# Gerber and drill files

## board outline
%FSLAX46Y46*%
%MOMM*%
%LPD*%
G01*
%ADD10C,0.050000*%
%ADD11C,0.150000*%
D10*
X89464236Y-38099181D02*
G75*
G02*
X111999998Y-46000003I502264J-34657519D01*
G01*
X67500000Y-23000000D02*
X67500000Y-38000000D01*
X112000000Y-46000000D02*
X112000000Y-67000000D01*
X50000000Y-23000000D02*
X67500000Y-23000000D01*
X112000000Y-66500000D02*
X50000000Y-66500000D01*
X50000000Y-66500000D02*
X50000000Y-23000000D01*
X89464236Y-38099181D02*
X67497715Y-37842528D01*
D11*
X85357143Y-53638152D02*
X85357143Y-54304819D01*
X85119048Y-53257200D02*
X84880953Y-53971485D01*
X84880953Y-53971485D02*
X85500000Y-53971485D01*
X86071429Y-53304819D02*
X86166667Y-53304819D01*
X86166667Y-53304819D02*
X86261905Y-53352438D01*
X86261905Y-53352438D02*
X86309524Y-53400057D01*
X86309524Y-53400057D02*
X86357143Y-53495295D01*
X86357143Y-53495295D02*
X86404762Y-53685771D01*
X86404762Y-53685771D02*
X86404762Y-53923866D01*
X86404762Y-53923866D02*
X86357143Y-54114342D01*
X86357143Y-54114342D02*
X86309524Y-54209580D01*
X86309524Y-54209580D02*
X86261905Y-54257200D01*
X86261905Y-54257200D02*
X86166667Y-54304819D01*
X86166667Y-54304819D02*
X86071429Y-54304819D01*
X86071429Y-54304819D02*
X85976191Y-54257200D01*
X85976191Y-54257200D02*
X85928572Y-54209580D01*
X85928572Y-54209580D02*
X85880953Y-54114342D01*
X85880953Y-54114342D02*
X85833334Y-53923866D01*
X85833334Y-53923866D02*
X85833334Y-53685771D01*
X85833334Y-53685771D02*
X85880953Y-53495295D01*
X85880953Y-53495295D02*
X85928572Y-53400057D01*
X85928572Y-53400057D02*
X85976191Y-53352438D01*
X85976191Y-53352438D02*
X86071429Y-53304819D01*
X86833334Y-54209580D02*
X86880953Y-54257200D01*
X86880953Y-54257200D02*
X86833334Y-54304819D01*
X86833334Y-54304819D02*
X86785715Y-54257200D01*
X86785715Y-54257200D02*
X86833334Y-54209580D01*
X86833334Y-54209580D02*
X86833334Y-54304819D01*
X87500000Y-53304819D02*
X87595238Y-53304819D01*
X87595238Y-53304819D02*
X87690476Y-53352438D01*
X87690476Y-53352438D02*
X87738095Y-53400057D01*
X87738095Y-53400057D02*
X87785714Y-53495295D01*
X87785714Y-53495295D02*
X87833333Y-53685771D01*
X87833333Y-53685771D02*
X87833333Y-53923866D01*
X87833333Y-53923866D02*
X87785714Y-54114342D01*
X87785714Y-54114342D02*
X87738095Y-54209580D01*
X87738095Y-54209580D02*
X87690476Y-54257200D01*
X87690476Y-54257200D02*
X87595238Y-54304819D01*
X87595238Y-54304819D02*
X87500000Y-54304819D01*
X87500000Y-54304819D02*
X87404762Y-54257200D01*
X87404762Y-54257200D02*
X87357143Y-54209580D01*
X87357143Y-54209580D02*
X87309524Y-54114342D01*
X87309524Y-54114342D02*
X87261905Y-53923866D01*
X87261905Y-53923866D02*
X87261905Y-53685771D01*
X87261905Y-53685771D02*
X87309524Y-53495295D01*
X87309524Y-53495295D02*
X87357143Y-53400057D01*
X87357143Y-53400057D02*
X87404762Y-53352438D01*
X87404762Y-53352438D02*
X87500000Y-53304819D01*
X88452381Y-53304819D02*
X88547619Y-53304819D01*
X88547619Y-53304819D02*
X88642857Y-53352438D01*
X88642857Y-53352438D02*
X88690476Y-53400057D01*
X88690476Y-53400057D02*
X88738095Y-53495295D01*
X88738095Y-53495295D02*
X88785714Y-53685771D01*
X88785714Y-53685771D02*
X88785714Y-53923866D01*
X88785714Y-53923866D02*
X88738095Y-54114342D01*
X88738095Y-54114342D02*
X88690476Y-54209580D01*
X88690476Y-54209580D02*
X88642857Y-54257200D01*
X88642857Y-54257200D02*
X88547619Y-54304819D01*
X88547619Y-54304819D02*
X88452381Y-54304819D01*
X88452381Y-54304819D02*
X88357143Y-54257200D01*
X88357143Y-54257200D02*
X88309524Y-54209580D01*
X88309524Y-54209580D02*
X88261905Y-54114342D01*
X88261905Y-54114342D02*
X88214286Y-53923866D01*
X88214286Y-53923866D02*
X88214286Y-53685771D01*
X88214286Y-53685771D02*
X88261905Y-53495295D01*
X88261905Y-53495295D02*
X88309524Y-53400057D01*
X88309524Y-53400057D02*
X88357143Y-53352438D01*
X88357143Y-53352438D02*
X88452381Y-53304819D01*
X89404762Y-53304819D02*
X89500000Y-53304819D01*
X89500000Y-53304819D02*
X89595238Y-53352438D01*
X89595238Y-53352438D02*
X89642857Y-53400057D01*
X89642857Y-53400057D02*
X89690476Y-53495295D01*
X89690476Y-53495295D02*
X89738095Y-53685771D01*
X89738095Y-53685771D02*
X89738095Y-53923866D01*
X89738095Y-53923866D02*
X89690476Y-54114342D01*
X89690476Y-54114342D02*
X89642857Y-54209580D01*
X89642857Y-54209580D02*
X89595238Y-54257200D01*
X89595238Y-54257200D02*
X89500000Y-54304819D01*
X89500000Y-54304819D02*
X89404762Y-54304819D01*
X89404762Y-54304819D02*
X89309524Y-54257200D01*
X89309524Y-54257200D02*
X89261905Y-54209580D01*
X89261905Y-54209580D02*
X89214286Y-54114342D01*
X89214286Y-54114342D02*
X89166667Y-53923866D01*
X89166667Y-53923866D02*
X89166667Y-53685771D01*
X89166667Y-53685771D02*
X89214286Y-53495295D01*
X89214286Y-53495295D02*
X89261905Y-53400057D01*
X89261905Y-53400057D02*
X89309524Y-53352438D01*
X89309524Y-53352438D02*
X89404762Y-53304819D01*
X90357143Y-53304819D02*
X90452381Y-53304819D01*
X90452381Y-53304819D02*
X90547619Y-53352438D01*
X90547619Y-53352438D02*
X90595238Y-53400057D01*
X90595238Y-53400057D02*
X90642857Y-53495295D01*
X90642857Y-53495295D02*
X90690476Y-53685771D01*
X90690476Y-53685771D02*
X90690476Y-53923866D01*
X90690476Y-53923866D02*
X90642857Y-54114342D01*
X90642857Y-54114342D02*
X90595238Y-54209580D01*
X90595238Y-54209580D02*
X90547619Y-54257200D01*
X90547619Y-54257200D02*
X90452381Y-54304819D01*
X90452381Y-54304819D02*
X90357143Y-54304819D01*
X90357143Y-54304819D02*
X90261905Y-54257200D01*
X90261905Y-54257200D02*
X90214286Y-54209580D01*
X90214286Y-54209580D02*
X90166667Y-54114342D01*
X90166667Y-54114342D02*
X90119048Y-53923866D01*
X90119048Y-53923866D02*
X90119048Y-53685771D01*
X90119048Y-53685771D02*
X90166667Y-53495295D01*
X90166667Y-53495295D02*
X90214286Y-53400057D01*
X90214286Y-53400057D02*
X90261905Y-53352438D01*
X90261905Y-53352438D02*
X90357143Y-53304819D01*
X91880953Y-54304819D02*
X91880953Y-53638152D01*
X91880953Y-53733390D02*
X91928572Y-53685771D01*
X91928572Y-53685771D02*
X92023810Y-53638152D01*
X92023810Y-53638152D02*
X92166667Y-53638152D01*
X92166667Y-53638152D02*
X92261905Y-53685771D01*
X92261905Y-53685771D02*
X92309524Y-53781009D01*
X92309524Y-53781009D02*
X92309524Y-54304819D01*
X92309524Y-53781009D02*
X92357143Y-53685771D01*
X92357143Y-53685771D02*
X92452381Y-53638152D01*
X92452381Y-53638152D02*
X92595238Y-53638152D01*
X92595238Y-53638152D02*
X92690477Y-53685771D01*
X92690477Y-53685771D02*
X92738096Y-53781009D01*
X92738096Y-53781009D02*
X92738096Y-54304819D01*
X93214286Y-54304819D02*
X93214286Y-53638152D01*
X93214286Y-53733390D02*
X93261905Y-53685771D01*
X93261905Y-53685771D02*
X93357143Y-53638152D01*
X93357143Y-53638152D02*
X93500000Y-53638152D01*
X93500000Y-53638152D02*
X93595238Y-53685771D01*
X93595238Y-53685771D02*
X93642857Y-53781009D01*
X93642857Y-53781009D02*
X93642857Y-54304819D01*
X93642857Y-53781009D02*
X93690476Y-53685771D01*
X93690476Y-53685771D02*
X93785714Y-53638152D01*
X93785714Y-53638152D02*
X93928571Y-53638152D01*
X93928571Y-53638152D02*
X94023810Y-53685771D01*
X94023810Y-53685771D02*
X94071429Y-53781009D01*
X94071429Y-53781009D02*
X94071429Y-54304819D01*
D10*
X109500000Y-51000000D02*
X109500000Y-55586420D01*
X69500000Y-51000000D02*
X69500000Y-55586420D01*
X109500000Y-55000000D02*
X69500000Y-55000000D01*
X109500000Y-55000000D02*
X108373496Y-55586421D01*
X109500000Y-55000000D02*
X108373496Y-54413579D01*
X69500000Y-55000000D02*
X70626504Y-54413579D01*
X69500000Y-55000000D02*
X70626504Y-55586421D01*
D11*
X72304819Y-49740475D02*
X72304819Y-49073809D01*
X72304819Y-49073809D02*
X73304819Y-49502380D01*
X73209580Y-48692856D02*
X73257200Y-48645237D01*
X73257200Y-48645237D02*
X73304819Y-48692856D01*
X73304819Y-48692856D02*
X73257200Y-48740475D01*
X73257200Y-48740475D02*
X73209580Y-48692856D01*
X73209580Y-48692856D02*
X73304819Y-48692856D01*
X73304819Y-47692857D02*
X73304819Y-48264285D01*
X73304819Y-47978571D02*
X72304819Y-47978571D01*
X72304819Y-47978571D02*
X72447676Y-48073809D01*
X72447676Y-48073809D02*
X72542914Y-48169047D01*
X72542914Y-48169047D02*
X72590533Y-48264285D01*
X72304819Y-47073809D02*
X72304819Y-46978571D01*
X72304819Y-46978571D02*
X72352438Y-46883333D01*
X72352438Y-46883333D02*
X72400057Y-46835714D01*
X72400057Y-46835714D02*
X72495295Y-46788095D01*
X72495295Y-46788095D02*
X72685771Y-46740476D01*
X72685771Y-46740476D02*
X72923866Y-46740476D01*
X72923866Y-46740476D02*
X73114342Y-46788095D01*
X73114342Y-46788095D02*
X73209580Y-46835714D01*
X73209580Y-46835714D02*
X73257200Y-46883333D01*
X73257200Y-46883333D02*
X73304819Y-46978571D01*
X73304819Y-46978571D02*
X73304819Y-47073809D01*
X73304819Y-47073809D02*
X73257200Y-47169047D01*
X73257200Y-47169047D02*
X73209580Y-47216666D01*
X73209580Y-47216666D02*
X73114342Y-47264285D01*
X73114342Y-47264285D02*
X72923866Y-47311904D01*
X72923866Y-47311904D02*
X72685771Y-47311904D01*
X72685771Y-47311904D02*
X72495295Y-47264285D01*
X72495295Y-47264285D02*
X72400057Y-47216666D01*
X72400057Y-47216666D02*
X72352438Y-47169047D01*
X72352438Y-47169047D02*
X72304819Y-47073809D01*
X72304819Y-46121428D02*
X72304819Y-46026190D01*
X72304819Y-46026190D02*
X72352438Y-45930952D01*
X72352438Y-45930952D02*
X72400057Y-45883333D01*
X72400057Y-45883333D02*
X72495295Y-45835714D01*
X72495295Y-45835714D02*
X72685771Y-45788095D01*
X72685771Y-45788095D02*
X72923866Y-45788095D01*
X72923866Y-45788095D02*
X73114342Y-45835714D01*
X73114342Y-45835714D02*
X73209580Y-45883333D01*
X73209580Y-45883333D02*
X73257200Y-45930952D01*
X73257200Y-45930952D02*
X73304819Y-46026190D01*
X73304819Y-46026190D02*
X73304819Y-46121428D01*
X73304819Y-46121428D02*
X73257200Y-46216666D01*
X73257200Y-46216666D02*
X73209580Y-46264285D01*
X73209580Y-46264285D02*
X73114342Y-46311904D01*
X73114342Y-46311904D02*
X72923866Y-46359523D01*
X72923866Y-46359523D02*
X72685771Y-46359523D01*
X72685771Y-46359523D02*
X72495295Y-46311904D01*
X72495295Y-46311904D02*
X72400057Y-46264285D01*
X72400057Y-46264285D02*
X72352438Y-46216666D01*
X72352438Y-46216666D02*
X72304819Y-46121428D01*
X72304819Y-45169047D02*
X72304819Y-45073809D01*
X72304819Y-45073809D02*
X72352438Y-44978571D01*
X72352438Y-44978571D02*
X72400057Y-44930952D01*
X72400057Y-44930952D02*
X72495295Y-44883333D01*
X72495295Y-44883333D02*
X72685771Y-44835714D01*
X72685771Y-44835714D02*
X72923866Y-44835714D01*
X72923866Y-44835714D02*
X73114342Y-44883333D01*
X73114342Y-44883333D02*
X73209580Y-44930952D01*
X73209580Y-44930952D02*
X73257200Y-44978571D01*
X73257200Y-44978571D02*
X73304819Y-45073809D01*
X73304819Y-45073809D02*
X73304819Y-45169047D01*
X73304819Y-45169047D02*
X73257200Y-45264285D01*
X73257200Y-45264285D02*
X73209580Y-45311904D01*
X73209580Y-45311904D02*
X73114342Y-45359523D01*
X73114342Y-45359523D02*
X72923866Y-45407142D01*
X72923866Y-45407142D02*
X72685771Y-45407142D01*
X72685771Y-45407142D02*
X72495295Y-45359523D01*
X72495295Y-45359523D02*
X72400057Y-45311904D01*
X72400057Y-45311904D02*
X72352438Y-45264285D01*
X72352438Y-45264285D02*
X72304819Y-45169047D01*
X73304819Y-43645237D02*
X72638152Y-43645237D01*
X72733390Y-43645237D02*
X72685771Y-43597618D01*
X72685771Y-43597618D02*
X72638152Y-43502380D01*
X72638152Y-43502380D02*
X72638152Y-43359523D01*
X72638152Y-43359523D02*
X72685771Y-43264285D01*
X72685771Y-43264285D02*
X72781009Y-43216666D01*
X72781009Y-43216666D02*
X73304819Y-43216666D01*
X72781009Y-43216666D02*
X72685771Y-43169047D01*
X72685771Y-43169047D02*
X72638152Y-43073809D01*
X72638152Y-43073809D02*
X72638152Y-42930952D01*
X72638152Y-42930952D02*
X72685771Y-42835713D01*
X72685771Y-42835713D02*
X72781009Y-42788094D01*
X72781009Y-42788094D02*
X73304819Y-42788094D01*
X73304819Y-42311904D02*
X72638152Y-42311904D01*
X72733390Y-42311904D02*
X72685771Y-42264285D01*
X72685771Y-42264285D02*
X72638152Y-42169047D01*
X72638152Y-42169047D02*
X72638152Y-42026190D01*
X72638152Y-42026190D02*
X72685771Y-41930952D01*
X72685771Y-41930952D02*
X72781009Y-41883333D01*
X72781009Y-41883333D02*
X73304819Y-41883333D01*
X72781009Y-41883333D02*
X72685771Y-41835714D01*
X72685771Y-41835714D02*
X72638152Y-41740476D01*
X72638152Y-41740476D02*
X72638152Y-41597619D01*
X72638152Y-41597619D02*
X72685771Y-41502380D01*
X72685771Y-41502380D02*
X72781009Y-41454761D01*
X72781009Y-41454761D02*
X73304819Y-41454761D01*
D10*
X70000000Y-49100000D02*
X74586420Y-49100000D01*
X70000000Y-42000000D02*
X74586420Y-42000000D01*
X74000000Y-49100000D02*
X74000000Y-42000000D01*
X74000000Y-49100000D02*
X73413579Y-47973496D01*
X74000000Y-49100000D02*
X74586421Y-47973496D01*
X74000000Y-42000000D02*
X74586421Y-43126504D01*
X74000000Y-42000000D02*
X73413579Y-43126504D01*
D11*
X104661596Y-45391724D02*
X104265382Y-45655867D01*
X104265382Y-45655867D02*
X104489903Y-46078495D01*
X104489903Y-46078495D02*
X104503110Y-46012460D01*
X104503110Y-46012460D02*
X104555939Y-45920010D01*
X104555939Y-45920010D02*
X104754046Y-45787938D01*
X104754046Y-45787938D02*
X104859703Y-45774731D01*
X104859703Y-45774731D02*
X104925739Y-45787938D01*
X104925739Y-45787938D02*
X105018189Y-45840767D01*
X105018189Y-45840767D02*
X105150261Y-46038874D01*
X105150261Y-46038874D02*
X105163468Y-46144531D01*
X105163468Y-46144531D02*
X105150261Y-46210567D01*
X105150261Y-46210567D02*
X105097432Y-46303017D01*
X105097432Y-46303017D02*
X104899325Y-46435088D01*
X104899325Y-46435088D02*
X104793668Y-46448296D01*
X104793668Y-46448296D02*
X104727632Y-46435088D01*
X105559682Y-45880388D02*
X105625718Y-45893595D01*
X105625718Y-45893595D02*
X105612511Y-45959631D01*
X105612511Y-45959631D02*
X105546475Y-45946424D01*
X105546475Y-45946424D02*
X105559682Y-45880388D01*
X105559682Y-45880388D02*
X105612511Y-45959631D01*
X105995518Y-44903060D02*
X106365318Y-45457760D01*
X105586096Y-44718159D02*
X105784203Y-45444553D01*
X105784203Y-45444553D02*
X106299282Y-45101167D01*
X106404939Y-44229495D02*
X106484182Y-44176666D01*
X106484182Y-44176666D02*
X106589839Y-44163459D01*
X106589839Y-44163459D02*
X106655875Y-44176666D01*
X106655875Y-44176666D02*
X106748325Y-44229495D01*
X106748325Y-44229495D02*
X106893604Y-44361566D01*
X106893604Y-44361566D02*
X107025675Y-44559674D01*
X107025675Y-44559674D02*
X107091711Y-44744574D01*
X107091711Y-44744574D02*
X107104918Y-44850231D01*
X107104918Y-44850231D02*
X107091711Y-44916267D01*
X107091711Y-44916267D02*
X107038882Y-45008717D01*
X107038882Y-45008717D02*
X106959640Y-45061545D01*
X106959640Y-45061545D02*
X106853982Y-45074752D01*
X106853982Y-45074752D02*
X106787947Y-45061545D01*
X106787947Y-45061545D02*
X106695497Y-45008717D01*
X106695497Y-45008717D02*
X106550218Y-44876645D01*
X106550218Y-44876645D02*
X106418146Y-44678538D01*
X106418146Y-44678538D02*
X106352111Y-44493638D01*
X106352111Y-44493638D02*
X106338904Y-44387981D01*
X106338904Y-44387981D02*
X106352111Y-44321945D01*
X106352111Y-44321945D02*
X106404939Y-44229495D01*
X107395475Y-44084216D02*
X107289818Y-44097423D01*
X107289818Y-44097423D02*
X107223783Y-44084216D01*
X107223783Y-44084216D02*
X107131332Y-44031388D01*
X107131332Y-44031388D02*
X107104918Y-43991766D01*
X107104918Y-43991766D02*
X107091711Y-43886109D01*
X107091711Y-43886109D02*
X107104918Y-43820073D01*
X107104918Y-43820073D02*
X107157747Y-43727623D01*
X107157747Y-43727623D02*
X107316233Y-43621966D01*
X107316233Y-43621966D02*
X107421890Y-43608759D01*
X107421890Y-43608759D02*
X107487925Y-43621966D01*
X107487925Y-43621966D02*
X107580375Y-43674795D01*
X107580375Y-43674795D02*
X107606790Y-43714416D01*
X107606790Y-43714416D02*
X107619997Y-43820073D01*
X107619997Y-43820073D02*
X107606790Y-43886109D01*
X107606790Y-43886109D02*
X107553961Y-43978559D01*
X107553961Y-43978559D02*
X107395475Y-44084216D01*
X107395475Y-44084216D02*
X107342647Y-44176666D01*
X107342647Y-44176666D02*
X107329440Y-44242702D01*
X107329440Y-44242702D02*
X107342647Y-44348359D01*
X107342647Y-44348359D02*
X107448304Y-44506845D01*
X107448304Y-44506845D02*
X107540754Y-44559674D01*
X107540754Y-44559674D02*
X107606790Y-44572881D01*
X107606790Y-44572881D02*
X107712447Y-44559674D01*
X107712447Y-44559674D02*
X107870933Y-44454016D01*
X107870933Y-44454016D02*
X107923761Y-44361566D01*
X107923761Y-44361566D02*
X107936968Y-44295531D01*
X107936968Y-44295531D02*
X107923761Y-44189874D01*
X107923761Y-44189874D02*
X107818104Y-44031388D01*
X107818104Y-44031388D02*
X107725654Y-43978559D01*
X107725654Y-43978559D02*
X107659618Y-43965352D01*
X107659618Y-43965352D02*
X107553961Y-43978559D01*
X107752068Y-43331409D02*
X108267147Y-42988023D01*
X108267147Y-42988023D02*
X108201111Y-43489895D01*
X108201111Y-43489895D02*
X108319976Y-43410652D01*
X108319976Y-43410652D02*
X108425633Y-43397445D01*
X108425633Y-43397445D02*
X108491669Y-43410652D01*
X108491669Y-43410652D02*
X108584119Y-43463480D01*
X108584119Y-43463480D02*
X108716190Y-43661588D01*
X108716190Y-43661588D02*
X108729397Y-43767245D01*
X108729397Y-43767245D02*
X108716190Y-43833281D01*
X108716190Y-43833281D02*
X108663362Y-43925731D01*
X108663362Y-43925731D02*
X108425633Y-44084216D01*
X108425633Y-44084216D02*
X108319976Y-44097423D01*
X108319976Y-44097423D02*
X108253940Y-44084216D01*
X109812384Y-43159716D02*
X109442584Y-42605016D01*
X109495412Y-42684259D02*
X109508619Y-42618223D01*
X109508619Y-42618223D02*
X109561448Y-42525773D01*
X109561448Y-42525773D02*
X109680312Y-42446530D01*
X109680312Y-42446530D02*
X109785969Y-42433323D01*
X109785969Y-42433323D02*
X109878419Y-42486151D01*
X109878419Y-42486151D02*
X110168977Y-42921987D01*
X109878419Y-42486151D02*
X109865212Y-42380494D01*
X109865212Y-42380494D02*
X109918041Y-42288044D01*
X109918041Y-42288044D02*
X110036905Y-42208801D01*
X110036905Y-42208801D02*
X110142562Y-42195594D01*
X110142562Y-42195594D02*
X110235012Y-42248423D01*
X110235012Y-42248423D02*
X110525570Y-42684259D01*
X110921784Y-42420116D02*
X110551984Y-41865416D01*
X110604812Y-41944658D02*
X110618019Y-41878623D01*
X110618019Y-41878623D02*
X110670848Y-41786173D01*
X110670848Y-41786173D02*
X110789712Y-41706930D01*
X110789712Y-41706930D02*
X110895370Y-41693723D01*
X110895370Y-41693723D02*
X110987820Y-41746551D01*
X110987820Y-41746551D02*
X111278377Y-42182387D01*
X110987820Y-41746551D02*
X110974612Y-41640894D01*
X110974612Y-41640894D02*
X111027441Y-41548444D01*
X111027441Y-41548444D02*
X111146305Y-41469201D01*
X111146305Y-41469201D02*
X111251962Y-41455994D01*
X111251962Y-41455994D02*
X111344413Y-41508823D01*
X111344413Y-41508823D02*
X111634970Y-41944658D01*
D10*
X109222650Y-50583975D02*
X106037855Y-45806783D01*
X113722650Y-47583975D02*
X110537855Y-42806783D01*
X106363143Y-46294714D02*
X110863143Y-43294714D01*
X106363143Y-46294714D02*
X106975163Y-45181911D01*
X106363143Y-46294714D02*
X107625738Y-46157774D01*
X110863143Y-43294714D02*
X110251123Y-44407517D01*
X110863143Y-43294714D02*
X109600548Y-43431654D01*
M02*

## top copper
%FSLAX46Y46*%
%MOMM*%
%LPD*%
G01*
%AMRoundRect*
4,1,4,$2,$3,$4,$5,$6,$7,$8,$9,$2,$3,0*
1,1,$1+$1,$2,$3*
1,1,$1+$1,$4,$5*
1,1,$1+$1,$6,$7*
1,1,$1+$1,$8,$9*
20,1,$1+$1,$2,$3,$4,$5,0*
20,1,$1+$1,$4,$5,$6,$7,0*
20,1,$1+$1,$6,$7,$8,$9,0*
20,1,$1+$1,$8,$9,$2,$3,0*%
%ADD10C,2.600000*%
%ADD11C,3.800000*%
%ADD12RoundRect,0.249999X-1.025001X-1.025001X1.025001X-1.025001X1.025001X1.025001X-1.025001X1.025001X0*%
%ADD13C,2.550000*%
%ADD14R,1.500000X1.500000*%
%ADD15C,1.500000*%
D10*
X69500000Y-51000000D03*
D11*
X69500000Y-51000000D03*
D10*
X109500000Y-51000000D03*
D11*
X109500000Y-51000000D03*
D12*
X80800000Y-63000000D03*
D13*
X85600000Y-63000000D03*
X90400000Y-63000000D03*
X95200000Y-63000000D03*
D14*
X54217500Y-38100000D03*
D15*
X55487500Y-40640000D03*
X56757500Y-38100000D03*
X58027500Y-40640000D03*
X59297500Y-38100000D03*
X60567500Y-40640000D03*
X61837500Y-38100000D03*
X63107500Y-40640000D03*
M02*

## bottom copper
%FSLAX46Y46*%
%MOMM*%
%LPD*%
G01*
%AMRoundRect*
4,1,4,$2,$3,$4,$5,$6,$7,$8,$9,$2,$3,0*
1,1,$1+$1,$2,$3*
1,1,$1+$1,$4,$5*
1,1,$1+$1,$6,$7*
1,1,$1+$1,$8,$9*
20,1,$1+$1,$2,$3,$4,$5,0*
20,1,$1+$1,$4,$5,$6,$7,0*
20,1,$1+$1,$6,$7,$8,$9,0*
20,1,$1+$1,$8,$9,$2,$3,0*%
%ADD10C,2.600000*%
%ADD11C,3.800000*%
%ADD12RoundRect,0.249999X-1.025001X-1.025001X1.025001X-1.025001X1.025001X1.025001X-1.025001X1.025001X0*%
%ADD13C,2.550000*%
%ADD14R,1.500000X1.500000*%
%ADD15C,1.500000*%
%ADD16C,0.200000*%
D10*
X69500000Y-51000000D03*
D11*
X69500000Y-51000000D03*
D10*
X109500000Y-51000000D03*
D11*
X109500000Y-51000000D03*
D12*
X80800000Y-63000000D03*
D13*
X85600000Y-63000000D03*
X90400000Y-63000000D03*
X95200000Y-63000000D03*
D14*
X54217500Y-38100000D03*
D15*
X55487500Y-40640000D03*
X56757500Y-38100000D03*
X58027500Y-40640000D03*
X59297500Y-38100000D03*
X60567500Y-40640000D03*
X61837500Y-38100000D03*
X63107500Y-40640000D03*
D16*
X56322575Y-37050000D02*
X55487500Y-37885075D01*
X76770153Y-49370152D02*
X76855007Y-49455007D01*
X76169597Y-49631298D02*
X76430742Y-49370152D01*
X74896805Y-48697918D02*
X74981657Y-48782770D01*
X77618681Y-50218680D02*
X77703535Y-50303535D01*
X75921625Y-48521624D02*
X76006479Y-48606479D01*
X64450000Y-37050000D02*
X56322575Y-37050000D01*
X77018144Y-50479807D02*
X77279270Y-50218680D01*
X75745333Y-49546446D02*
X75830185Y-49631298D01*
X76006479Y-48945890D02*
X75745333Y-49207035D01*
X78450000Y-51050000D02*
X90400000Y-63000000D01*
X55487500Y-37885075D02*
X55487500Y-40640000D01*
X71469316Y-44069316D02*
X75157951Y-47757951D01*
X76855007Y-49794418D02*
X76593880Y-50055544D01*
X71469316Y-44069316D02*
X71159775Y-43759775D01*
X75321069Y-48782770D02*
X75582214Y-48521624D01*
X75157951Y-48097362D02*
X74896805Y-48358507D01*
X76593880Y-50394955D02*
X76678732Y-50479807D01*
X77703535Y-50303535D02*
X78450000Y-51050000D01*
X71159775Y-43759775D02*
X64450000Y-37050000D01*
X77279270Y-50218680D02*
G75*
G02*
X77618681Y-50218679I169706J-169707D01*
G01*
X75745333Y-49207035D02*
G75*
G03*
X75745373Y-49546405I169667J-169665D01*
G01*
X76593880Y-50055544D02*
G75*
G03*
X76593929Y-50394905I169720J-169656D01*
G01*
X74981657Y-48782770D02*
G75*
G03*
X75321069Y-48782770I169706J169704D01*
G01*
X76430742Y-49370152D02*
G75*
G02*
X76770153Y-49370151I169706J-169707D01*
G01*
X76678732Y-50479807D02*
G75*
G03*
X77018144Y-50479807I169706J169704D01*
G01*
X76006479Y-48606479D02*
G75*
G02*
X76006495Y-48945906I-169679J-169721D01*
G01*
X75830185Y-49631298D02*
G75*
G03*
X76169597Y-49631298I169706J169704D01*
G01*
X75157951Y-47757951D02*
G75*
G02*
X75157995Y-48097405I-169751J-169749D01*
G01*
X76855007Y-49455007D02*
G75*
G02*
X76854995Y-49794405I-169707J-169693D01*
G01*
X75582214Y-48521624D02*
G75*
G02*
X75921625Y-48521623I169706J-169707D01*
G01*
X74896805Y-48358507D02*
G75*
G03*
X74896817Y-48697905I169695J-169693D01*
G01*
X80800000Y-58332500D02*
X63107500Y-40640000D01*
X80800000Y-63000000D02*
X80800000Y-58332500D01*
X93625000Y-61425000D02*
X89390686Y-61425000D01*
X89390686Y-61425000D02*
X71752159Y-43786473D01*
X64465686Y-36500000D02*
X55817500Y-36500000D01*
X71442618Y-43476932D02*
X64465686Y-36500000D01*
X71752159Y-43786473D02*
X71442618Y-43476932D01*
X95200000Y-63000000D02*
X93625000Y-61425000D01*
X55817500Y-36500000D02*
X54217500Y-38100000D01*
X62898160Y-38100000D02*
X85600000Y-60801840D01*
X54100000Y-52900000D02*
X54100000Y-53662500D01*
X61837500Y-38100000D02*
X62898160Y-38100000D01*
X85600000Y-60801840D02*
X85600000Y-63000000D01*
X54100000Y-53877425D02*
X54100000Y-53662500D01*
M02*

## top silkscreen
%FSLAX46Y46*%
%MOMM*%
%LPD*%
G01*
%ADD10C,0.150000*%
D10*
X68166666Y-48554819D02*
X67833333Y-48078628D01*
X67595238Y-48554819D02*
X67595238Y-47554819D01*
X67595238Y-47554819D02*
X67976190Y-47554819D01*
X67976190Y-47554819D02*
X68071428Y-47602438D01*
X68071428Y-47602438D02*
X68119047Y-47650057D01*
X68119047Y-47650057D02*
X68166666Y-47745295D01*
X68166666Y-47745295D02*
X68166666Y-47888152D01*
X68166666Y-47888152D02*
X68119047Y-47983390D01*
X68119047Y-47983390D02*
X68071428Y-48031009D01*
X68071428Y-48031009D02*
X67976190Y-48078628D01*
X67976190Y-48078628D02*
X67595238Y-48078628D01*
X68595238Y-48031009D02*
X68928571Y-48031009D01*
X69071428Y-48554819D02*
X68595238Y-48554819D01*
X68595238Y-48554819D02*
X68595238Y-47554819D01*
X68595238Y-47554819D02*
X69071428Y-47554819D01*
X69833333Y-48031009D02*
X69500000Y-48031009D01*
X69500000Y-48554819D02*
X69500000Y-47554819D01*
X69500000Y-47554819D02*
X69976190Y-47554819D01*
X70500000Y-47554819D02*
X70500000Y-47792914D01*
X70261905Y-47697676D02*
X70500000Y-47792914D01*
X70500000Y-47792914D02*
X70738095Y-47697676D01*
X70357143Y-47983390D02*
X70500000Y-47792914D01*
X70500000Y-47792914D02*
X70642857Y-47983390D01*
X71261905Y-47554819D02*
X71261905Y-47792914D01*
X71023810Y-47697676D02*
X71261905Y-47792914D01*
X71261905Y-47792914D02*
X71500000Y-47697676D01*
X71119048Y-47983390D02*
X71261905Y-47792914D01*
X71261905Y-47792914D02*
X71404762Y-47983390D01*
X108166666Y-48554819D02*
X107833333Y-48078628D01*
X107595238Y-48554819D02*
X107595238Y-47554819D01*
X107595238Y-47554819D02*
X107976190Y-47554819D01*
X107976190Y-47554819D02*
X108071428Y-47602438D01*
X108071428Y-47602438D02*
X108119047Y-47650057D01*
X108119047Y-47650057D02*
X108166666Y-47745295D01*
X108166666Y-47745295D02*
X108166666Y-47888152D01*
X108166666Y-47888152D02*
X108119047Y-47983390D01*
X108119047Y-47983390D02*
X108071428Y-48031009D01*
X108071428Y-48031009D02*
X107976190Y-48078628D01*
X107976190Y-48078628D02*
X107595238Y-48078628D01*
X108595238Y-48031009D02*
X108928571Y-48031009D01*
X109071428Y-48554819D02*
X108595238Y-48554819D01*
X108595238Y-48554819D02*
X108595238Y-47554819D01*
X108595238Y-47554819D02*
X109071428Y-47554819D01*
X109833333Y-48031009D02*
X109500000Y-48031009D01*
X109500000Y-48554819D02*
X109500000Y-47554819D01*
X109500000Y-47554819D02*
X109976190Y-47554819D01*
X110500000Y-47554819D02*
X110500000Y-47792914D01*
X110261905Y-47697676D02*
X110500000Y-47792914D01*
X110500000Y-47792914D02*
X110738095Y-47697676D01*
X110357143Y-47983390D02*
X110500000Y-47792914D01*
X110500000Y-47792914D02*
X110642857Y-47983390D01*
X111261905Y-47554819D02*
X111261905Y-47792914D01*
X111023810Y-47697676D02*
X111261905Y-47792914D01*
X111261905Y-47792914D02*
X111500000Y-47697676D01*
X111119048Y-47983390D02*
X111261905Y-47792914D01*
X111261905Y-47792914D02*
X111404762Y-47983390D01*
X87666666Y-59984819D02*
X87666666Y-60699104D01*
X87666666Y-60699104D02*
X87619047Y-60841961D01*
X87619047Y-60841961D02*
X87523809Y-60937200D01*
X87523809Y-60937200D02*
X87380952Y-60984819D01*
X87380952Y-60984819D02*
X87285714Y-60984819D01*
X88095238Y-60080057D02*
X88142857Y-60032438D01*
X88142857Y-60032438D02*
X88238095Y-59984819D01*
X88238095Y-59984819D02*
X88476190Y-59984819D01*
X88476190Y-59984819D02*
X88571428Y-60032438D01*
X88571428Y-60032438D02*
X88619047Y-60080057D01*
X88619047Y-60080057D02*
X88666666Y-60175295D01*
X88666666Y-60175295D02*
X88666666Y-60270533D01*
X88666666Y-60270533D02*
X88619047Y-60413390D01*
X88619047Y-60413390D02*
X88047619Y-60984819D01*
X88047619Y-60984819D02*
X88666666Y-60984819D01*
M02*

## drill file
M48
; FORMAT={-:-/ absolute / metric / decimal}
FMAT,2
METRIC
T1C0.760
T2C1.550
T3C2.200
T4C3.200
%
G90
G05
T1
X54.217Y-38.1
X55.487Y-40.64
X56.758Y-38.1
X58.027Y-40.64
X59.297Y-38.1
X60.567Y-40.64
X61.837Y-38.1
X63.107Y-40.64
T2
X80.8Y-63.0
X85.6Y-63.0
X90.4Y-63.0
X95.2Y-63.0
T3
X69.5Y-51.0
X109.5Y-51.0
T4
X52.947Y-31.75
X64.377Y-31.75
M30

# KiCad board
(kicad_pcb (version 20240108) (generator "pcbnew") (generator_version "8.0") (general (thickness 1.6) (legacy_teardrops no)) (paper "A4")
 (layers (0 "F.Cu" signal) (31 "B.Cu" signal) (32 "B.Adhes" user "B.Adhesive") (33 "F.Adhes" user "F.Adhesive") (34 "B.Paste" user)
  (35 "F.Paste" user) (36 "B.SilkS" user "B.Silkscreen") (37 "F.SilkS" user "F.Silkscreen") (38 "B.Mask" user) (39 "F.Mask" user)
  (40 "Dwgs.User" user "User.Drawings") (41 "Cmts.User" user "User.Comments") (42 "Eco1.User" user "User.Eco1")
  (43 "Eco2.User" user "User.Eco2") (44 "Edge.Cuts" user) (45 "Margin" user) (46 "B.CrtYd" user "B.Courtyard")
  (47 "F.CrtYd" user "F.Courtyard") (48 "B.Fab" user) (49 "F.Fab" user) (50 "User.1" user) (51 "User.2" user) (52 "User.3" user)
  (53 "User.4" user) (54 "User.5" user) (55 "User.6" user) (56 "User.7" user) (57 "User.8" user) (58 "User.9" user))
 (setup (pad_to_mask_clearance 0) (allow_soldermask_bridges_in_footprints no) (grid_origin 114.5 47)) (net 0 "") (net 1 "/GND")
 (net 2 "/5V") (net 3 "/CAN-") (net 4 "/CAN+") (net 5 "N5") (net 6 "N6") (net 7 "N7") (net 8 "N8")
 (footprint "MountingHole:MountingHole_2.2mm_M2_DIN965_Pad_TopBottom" (layer "F.Cu") (at 69.5 51)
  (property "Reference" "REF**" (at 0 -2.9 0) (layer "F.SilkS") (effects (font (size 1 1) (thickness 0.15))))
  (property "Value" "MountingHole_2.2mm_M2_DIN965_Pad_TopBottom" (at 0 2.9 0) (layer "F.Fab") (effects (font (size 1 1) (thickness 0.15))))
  (pad "1" thru_hole circle (at 0 0) (size 2.6 2.6) (drill 2.2) (layers "*.Cu" "*.Mask") (remove_unused_layers no))
  (pad "1" connect circle (at 0 0) (size 3.8 3.8) (layers "F.Cu" "F.Mask"))
  (pad "1" connect circle (at 0 0) (size 3.8 3.8) (layers "B.Cu" "B.Mask")))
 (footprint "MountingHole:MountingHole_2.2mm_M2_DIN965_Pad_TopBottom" (layer "F.Cu") (at 109.5 51)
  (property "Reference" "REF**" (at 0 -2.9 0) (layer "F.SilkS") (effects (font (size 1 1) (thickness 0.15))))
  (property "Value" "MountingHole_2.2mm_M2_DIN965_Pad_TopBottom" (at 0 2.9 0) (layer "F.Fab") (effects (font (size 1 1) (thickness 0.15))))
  (pad "1" thru_hole circle (at 0 0) (size 2.6 2.6) (drill 2.2) (layers "*.Cu" "*.Mask") (remove_unused_layers no))
  (pad "1" connect circle (at 0 0) (size 3.8 3.8) (layers "F.Cu" "F.Mask"))
  (pad "1" connect circle (at 0 0) (size 3.8 3.8) (layers "B.Cu" "B.Mask")))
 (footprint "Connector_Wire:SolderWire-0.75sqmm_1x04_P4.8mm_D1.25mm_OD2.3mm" (layer "F.Cu") (at 80.8 63)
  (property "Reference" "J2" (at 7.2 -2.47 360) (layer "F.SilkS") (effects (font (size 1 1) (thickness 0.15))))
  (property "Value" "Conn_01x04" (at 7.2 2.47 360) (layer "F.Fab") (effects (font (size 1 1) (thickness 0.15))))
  (pad "1" thru_hole roundrect (at 0 0) (size 2.55 2.55) (drill 1.55) (layers "*.Cu" "*.Mask") (remove_unused_layers no)
   (roundrect_rratio 0.098039) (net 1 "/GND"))
  (pad "2" thru_hole circle (at 4.8 0) (size 2.55 2.55) (drill 1.55) (layers "*.Cu" "*.Mask") (remove_unused_layers no) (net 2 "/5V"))
  (pad "3" thru_hole circle (at 9.6 0) (size 2.55 2.55) (drill 1.55) (layers "*.Cu" "*.Mask") (remove_unused_layers no) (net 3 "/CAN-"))
  (pad "4" thru_hole circle (at 14.4 0) (size 2.55 2.55) (drill 1.55) (layers "*.Cu" "*.Mask") (remove_unused_layers no) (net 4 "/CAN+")))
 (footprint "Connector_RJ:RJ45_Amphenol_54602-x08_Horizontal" (layer "B.Cu") (at 54.2175 38.1)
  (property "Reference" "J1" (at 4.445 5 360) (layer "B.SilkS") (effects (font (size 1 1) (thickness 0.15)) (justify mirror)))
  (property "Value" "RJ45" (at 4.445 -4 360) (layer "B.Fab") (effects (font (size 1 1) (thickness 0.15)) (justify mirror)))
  (pad "" np_thru_hole circle (at -1.27 -6.35) (size 3.2 3.2) (drill 3.2) (layers "*.Cu" "*.Mask"))
  (pad "" np_thru_hole circle (at 10.16 -6.35) (size 3.2 3.2) (drill 3.2) (layers "*.Cu" "*.Mask"))
  (pad "1" thru_hole rect (at 0 0) (size 1.5 1.5) (drill 0.76) (layers "*.Cu" "*.Mask") (remove_unused_layers no) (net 4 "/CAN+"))
  (pad "2" thru_hole circle (at 1.27 2.54) (size 1.5 1.5) (drill 0.76) (layers "*.Cu" "*.Mask") (remove_unused_layers no) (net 3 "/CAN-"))
  (pad "3" thru_hole circle (at 2.54 0) (size 1.5 1.5) (drill 0.76) (layers "*.Cu" "*.Mask") (remove_unused_layers no) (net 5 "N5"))
  (pad "4" thru_hole circle (at 3.81 2.54) (size 1.5 1.5) (drill 0.76) (layers "*.Cu" "*.Mask") (remove_unused_layers no) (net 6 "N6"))
  (pad "5" thru_hole circle (at 5.08 0) (size 1.5 1.5) (drill 0.76) (layers "*.Cu" "*.Mask") (remove_unused_layers no) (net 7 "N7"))
  (pad "6" thru_hole circle (at 6.35 2.54) (size 1.5 1.5) (drill 0.76) (layers "*.Cu" "*.Mask") (remove_unused_layers no) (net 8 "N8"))
  (pad "7" thru_hole circle (at 7.62 0) (size 1.5 1.5) (drill 0.76) (layers "*.Cu" "*.Mask") (remove_unused_layers no) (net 2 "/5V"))
  (pad "8" thru_hole circle (at 8.89 2.54) (size 1.5 1.5) (drill 0.76) (layers "*.Cu" "*.Mask") (remove_unused_layers no) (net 1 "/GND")))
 (gr_arc (start 89.464236 38.099181) (mid 101.434032 40.047498) (end 112 46) (stroke (width 0.05) (type default)) (layer "Edge.Cuts"))
 (gr_line (start 67.5 23) (end 67.5 38) (stroke (width 0.05) (type default)) (layer "Edge.Cuts"))
 (gr_line (start 112 46) (end 112 67) (stroke (width 0.05) (type default)) (layer "Edge.Cuts"))
 (gr_line (start 50 23) (end 67.5 23) (stroke (width 0.05) (type default)) (layer "Edge.Cuts"))
 (gr_line (start 112 66.5) (end 50 66.5) (stroke (width 0.05) (type default)) (layer "Edge.Cuts"))
 (gr_line (start 50 66.5) (end 50 23) (stroke (width 0.05) (type default)) (layer "Edge.Cuts"))
 (gr_line (start 89.464236 38.099181) (end 67.497715 37.842528) (stroke (width 0.05) (type default)) (layer "Edge.Cuts"))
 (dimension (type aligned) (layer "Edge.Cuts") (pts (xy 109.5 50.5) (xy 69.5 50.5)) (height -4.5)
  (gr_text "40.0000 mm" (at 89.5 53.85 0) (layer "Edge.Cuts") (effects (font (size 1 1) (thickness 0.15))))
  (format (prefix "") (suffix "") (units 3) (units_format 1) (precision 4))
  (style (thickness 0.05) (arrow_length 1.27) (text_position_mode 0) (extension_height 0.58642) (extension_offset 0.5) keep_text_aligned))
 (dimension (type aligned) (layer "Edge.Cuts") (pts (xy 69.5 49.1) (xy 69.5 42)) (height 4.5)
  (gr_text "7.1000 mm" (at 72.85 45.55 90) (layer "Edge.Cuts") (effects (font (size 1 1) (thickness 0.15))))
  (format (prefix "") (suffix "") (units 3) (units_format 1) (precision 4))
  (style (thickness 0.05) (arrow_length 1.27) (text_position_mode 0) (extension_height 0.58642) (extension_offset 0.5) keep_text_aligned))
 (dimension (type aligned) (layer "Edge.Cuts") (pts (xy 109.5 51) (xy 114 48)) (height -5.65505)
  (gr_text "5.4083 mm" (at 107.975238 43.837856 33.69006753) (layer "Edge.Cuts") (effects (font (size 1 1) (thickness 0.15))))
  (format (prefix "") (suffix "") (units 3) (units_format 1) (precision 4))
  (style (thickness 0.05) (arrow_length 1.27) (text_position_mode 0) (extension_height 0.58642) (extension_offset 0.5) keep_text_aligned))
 (segment (start 56.322575 37.05) (end 55.4875 37.885075) (width 0.2) (layer "B.Cu") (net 3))
 (segment (start 76.770153 49.370152) (end 76.855007 49.455007) (width 0.2) (layer "B.Cu") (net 3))
 (segment (start 76.169597 49.631298) (end 76.430742 49.370152) (width 0.2) (layer "B.Cu") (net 3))
 (segment (start 74.896805 48.697918) (end 74.981657 48.78277) (width 0.2) (layer "B.Cu") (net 3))
 (segment (start 77.618681 50.21868) (end 77.703535 50.303535) (width 0.2) (layer "B.Cu") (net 3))
 (segment (start 75.921625 48.521624) (end 76.006479 48.606479) (width 0.2) (layer "B.Cu") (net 3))
 (segment (start 64.45 37.05) (end 56.322575 37.05) (width 0.2) (layer "B.Cu") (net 3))
 (segment (start 77.018144 50.479807) (end 77.27927 50.21868) (width 0.2) (layer "B.Cu") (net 3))
 (segment (start 75.745333 49.546446) (end 75.830185 49.631298) (width 0.2) (layer "B.Cu") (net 3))
 (segment (start 76.006479 48.94589) (end 75.745333 49.207035) (width 0.2) (layer "B.Cu") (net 3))
 (segment (start 78.45 51.05) (end 90.4 63) (width 0.2) (layer "B.Cu") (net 3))
 (segment (start 55.4875 37.885075) (end 55.4875 40.64) (width 0.2) (layer "B.Cu") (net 3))
 (segment (start 71.469316 44.069316) (end 75.157951 47.757951) (width 0.2) (layer "B.Cu") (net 3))
 (segment (start 76.855007 49.794418) (end 76.59388 50.055544) (width 0.2) (layer "B.Cu") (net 3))
 (segment (start 71.469316 44.069316) (end 71.159775 43.759775) (width 0.2) (layer "B.Cu") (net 3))
 (segment (start 75.321069 48.78277) (end 75.582214 48.521624) (width 0.2) (layer "B.Cu") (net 3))
 (segment (start 75.157951 48.097362) (end 74.896805 48.358507) (width 0.2) (layer "B.Cu") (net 3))
 (segment (start 76.59388 50.394955) (end 76.678732 50.479807) (width 0.2) (layer "B.Cu") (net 3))
 (segment (start 77.703535 50.303535) (end 78.45 51.05) (width 0.2) (layer "B.Cu") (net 3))
 (segment (start 71.159775 43.759775) (end 64.45 37.05) (width 0.2) (layer "B.Cu") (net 3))
 (arc (start 77.27927 50.21868) (mid 77.448975 50.148386) (end 77.618681 50.21868) (width 0.2) (layer "B.Cu") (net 3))
 (arc (start 75.745333 49.207035) (mid 75.675039 49.37674) (end 75.745333 49.546446) (width 0.2) (layer "B.Cu") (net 3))
 (arc (start 76.59388 50.055544) (mid 76.523586 50.225249) (end 76.59388 50.394955) (width 0.2) (layer "B.Cu") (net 3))
 (arc (start 74.981657 48.78277) (mid 75.151363 48.853065) (end 75.321069 48.78277) (width 0.2) (layer "B.Cu") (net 3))
 (arc (start 76.430742 49.370152) (mid 76.600447 49.299858) (end 76.770153 49.370152) (width 0.2) (layer "B.Cu") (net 3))
 (arc (start 76.678732 50.479807) (mid 76.848438 50.550102) (end 77.018144 50.479807) (width 0.2) (layer "B.Cu") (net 3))
 (arc (start 76.006479 48.606479) (mid 76.076773 48.776185) (end 76.006479 48.94589) (width 0.2) (layer "B.Cu") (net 3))
 (arc (start 75.830185 49.631298) (mid 75.999891 49.701593) (end 76.169597 49.631298) (width 0.2) (layer "B.Cu") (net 3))
 (arc (start 75.157951 47.757951) (mid 75.228245 47.927657) (end 75.157951 48.097362) (width 0.2) (layer "B.Cu") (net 3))
 (arc (start 76.855007 49.455007) (mid 76.925301 49.624713) (end 76.855007 49.794418) (width 0.2) (layer "B.Cu") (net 3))
 (arc (start 75.582214 48.521624) (mid 75.751919 48.45133) (end 75.921625 48.521624) (width 0.2) (layer "B.Cu") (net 3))
 (arc (start 74.896805 48.358507) (mid 74.826511 48.528212) (end 74.896805 48.697918) (width 0.2) (layer "B.Cu") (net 3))
 (segment (start 80.8 58.3325) (end 63.1075 40.64) (width 0.2) (layer "B.Cu") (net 1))
 (segment (start 80.8 63) (end 80.8 58.3325) (width 0.2) (layer "B.Cu") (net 1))
 (segment (start 93.625 61.425) (end 89.390686 61.425) (width 0.2) (layer "B.Cu") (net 4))
 (segment (start 89.390686 61.425) (end 71.752159 43.786473) (width 0.2) (layer "B.Cu") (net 4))
 (segment (start 64.465686 36.5) (end 55.8175 36.5) (width 0.2) (layer "B.Cu") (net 4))
 (segment (start 71.442618 43.476932) (end 64.465686 36.5) (width 0.2) (layer "B.Cu") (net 4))
 (segment (start 71.752159 43.786473) (end 71.442618 43.476932) (width 0.2) (layer "B.Cu") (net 4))
 (segment (start 95.2 63) (end 93.625 61.425) (width 0.2) (layer "B.Cu") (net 4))
 (segment (start 55.8175 36.5) (end 54.2175 38.1) (width 0.2) (layer "B.Cu") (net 4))
 (segment (start 62.89816 38.1) (end 85.6 60.80184) (width 0.2) (layer "B.Cu") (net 2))
 (segment (start 54.1 52.9) (end 54.1 53.6625) (width 0.2) (layer "B.Cu") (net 2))
 (segment (start 61.8375 38.1) (end 62.89816 38.1) (width 0.2) (layer "B.Cu") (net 2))
 (segment (start 85.6 60.80184) (end 85.6 63) (width 0.2) (layer "B.Cu") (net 2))
 (segment (start 54.1 53.877425) (end 54.1 53.6625) (width 0.2) (layer "B.Cu") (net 2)))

